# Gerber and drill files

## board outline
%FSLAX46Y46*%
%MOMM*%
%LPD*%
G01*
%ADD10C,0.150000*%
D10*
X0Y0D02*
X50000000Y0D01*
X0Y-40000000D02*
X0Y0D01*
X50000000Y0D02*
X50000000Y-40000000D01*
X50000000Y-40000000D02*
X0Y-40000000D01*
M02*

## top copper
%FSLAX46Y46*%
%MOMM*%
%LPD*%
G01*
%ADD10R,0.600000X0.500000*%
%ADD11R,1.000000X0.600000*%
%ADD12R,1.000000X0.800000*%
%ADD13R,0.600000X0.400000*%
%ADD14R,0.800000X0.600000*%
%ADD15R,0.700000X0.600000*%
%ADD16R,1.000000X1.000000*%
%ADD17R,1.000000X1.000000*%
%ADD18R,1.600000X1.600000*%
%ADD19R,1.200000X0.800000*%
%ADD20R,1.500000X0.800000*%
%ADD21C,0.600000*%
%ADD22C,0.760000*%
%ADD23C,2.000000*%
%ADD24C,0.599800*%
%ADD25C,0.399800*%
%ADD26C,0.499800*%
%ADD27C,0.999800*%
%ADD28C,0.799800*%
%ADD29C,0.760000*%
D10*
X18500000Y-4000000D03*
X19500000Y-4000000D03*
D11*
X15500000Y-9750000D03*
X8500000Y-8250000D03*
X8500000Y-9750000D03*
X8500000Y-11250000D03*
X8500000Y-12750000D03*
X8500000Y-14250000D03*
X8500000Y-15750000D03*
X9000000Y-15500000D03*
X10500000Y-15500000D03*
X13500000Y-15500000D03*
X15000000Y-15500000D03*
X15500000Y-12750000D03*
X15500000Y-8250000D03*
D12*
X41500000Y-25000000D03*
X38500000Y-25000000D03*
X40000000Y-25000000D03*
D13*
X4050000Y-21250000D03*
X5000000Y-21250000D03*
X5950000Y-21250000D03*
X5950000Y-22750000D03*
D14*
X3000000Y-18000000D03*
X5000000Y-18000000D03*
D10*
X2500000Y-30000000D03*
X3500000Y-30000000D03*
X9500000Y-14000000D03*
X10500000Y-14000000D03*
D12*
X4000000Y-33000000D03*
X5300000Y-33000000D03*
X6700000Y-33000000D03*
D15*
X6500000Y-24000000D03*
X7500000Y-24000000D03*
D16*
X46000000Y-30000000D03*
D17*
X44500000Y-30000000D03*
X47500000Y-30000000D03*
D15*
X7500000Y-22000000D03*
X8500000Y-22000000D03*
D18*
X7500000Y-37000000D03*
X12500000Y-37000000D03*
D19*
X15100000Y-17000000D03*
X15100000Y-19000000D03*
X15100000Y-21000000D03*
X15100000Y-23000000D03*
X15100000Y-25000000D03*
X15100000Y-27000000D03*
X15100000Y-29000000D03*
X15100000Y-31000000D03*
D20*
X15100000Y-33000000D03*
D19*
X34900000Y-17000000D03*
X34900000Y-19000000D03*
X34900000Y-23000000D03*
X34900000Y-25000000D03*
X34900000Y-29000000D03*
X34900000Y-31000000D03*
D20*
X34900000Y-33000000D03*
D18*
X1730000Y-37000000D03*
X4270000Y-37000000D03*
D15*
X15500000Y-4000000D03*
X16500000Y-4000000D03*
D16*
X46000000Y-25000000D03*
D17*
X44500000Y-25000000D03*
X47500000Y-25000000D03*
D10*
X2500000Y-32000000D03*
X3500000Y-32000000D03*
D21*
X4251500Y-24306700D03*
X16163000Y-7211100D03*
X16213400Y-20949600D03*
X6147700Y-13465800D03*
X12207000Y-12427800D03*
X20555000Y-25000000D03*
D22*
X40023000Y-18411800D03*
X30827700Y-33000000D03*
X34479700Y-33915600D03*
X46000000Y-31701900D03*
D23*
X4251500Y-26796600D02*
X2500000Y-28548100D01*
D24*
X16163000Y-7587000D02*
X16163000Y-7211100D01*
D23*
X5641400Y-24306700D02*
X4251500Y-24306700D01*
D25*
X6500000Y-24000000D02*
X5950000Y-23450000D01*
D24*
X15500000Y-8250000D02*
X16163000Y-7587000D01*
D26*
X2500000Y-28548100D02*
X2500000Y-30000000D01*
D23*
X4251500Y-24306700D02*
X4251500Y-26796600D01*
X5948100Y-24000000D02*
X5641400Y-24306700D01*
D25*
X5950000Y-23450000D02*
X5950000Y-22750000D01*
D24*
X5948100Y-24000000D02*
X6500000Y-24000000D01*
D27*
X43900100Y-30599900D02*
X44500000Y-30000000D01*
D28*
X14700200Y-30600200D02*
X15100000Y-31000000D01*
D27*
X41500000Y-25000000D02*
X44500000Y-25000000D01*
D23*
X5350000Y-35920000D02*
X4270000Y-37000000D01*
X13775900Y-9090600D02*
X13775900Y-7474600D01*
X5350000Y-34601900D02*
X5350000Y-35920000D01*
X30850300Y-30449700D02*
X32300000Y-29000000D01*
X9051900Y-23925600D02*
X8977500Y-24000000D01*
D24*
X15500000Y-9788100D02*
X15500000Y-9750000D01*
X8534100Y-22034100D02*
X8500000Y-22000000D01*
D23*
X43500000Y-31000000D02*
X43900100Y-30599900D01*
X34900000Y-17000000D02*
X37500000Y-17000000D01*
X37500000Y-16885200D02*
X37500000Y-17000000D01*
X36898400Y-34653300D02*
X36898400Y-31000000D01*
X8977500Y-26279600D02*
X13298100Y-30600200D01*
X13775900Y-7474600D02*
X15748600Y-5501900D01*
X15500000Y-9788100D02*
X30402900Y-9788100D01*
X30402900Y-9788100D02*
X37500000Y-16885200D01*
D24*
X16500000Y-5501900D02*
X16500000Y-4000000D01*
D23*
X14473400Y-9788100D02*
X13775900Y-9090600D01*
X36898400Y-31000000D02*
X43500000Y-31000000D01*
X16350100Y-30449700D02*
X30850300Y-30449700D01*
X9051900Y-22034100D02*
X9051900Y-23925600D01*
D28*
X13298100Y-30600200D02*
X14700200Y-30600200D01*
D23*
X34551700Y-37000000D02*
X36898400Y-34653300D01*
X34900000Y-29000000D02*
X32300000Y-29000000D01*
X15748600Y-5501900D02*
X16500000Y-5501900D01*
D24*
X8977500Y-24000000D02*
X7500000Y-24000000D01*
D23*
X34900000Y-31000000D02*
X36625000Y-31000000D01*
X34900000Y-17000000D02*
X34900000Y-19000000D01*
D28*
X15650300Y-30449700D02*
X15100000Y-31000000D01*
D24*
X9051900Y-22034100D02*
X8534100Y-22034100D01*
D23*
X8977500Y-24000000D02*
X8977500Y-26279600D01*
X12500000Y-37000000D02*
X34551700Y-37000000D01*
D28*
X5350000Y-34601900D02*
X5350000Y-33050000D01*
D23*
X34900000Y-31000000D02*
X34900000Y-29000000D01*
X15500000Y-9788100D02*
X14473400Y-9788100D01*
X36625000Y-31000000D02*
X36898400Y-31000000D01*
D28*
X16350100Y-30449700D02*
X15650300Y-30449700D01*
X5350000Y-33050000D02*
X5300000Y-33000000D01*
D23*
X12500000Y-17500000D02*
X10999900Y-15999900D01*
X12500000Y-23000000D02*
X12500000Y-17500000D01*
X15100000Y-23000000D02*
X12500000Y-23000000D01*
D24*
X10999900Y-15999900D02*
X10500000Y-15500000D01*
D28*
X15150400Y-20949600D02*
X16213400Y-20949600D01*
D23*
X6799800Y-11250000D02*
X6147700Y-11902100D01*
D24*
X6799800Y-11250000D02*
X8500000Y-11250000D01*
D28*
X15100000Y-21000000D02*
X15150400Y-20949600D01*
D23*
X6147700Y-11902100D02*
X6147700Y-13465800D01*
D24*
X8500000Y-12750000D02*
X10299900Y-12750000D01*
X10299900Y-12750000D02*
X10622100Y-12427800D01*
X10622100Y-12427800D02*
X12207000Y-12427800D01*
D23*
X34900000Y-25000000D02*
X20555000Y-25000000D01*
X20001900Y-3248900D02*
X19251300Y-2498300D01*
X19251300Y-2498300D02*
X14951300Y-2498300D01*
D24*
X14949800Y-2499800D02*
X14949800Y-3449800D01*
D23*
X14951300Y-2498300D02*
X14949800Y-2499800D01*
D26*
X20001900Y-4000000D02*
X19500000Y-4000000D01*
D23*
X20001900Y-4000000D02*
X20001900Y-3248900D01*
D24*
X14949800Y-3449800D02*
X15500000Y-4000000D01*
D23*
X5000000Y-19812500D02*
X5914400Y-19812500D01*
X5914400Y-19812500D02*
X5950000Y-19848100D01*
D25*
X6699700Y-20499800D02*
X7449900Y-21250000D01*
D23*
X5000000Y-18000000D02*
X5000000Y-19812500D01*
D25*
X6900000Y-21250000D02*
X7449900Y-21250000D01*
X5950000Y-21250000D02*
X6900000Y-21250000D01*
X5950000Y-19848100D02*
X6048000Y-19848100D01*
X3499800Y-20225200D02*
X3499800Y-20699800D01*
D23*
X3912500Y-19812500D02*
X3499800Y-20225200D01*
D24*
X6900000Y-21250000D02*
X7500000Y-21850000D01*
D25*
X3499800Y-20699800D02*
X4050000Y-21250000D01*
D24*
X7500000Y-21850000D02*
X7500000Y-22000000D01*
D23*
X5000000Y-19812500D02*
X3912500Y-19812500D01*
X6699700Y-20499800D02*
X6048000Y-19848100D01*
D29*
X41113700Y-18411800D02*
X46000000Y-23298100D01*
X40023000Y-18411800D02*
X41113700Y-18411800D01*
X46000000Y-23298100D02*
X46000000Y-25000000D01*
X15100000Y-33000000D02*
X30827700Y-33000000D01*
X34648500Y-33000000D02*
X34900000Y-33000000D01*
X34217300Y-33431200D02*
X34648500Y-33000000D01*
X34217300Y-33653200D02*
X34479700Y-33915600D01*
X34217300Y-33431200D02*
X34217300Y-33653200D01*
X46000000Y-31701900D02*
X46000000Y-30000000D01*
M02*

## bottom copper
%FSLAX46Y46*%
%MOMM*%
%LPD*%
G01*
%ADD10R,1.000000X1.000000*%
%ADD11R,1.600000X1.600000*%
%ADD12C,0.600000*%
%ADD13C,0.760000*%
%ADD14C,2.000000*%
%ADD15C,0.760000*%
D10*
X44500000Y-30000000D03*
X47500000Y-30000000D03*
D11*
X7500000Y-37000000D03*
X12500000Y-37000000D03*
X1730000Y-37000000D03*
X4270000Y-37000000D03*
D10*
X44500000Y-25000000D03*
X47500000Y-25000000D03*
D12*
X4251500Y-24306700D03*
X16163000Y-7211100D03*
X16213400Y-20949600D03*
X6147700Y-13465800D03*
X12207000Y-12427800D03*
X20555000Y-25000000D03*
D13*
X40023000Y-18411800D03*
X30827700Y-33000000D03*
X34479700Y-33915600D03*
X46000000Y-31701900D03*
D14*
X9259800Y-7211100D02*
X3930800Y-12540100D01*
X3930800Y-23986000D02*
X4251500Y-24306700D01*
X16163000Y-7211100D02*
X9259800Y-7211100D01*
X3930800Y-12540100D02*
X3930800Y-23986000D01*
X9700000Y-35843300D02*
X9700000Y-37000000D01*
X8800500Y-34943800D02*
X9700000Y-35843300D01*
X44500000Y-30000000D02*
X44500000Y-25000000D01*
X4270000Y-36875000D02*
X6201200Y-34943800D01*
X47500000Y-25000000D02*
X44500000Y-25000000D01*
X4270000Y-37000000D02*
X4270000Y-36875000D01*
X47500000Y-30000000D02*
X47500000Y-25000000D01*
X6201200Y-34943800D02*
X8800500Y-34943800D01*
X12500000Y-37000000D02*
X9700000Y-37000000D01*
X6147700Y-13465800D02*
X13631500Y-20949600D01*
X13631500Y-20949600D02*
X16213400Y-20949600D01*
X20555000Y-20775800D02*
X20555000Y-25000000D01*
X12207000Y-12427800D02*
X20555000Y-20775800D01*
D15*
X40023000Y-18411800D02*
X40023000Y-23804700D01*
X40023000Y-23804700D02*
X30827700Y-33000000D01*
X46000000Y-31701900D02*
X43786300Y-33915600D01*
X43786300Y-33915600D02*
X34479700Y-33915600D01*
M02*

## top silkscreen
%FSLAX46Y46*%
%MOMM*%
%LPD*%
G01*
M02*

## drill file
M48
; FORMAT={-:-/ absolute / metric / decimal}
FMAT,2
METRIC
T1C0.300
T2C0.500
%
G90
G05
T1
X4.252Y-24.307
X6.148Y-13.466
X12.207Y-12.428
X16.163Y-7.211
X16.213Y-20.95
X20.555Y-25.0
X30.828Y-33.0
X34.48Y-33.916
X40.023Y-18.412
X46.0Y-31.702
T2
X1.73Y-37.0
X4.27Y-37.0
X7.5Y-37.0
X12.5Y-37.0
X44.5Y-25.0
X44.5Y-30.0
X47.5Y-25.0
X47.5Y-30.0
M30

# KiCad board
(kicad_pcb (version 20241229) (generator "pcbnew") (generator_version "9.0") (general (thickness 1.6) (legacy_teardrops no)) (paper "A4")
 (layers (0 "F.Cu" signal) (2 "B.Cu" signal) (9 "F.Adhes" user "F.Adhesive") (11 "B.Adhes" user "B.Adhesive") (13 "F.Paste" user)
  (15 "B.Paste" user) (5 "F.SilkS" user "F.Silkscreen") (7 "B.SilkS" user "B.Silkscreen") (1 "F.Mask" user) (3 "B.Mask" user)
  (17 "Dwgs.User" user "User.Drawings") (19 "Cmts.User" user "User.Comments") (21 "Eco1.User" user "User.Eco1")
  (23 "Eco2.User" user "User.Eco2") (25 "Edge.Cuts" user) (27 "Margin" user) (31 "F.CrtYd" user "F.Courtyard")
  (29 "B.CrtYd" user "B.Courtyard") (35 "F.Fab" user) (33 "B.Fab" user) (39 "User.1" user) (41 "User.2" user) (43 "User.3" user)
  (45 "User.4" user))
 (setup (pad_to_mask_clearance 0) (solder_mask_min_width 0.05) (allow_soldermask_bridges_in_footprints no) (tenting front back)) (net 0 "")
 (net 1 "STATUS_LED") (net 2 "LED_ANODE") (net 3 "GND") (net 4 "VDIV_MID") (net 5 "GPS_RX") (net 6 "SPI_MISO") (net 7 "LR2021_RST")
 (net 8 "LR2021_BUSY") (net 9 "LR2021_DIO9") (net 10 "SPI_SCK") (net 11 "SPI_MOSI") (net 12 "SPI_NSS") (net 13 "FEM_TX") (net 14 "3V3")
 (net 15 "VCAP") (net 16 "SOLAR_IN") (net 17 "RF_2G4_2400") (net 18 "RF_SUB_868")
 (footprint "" (layer "F.Cu") (at 19 4)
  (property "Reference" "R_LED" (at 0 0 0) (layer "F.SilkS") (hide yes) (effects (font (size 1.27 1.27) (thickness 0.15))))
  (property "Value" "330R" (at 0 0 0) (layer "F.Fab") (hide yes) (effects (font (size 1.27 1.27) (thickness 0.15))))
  (pad "1" smd rect (at -0.5 0) (size 0.6 0.5) (layers "F.Cu" "F.Mask") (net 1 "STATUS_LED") (thermal_bridge_angle 45))
  (pad "2" smd rect (at 0.5 0) (size 0.6 0.5) (layers "F.Cu" "F.Mask") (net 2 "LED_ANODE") (thermal_bridge_angle 45)))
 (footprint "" (layer "F.Cu") (at 12 12)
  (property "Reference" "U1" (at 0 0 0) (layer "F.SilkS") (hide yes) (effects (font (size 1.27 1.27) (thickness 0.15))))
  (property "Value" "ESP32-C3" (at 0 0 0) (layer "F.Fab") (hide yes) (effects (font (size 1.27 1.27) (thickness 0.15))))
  (pad "GND" smd rect (at 3.5 -2.25) (size 1 0.6) (layers "F.Cu" "F.Mask") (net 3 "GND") (thermal_bridge_angle 45))
  (pad "GPIO0" smd rect (at -3.5 -3.75) (size 1 0.6) (layers "F.Cu" "F.Mask") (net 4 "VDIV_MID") (thermal_bridge_angle 45))
  (pad "GPIO1" smd rect (at -3.5 -2.25) (size 1 0.6) (layers "F.Cu" "F.Mask") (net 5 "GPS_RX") (thermal_bridge_angle 45))
  (pad "GPIO2" smd rect (at -3.5 -0.75) (size 1 0.6) (layers "F.Cu" "F.Mask") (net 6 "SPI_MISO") (thermal_bridge_angle 45))
  (pad "GPIO3" smd rect (at -3.5 0.75) (size 1 0.6) (layers "F.Cu" "F.Mask") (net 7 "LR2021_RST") (thermal_bridge_angle 45))
  (pad "GPIO4" smd rect (at -3.5 2.25) (size 1 0.6) (layers "F.Cu" "F.Mask") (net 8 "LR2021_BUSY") (thermal_bridge_angle 45))
  (pad "GPIO5" smd rect (at -3.5 3.75) (size 1 0.6) (layers "F.Cu" "F.Mask") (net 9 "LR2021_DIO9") (thermal_bridge_angle 45))
  (pad "GPIO6" smd rect (at -3 3.5) (size 1 0.6) (layers "F.Cu" "F.Mask") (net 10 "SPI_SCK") (thermal_bridge_angle 45))
  (pad "GPIO7" smd rect (at -1.5 3.5) (size 1 0.6) (layers "F.Cu" "F.Mask") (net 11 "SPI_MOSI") (thermal_bridge_angle 45))
  (pad "GPIO9" smd rect (at 1.5 3.5) (size 1 0.6) (layers "F.Cu" "F.Mask") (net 1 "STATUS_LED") (thermal_bridge_angle 45))
  (pad "GPIO10" smd rect (at 3 3.5) (size 1 0.6) (layers "F.Cu" "F.Mask") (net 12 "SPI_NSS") (thermal_bridge_angle 45))
  (pad "GPIO19" smd rect (at 3.5 0.75) (size 1 0.6) (layers "F.Cu" "F.Mask") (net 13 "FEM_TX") (thermal_bridge_angle 45))
  (pad "VCC" smd rect (at 3.5 -3.75) (size 1 0.6) (layers "F.Cu" "F.Mask") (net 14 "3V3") (thermal_bridge_angle 45)))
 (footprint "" (layer "F.Cu") (at 40 25)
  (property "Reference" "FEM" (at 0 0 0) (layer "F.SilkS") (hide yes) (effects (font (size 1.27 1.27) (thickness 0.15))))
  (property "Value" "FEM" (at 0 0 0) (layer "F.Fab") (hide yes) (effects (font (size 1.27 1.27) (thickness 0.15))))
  (pad "GND" smd rect (at 1.5 0) (size 1 0.8) (layers "F.Cu" "F.Mask") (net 3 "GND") (thermal_bridge_angle 45))
  (pad "TX" smd rect (at -1.5 0) (size 1 0.8) (layers "F.Cu" "F.Mask") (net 13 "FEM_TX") (thermal_bridge_angle 45))
  (pad "VCC" smd rect (at 0 0) (size 1 0.8) (layers "F.Cu" "F.Mask") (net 14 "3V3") (thermal_bridge_angle 45)))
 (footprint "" (layer "F.Cu") (at 5 22)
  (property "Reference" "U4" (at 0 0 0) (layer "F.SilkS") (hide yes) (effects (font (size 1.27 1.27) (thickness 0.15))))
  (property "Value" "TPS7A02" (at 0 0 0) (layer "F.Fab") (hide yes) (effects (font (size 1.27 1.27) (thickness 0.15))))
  (pad "1" smd rect (at -0.95 -0.75) (size 0.6 0.4) (layers "F.Cu" "F.Mask") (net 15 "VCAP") (thermal_bridge_angle 45))
  (pad "2" smd rect (at 0 -0.75) (size 0.6 0.4) (layers "F.Cu" "F.Mask") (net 3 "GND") (thermal_bridge_angle 45))
  (pad "3" smd rect (at 0.95 -0.75) (size 0.6 0.4) (layers "F.Cu" "F.Mask") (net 15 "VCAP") (thermal_bridge_angle 45))
  (pad "4" smd rect (at 0.95 0.75) (size 0.6 0.4) (layers "F.Cu" "F.Mask") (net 14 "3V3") (thermal_bridge_angle 45)))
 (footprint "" (layer "F.Cu") (at 4 18)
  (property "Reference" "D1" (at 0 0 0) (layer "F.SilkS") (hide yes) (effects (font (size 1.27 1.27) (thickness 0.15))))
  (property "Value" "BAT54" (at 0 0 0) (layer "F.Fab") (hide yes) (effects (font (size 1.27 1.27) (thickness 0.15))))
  (pad "A" smd rect (at -1 0) (size 0.8 0.6) (layers "F.Cu" "F.Mask") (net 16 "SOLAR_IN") (thermal_bridge_angle 45))
  (pad "K" smd rect (at 1 0) (size 0.8 0.6) (layers "F.Cu" "F.Mask") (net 15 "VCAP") (thermal_bridge_angle 45)))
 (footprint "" (layer "F.Cu") (at 3 30)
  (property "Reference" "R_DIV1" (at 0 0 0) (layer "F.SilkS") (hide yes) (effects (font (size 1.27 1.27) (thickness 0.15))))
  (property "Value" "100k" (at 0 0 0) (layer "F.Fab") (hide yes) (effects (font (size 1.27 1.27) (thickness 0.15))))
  (pad "1" smd rect (at -0.5 0) (size 0.6 0.5) (layers "F.Cu" "F.Mask") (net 14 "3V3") (thermal_bridge_angle 45))
  (pad "2" smd rect (at 0.5 0) (size 0.6 0.5) (layers "F.Cu" "F.Mask") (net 4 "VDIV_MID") (thermal_bridge_angle 45)))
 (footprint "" (layer "F.Cu") (at 10 14)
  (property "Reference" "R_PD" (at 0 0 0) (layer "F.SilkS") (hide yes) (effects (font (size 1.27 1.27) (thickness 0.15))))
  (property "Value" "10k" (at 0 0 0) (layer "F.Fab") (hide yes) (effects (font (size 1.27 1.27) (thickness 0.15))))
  (pad "1" smd rect (at -0.5 0) (size 0.6 0.5) (layers "F.Cu" "F.Mask") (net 3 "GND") (thermal_bridge_angle 45))
  (pad "2" smd rect (at 0.5 0) (size 0.6 0.5) (layers "F.Cu" "F.Mask") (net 6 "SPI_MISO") (thermal_bridge_angle 45)))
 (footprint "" (layer "F.Cu") (at 6 33)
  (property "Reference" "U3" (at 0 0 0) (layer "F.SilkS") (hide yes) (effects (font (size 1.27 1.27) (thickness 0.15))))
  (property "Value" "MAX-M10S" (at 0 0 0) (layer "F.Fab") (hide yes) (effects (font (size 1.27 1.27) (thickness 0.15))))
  (pad "1" smd rect (at -2 0) (size 1 0.8) (layers "F.Cu" "F.Mask") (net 14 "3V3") (thermal_bridge_angle 45))
  (pad "2" smd rect (at -0.7 0) (size 1 0.8) (layers "F.Cu" "F.Mask") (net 3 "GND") (thermal_bridge_angle 45))
  (pad "3" smd rect (at 0.7 0) (size 1 0.8) (layers "F.Cu" "F.Mask") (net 5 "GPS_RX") (thermal_bridge_angle 45)))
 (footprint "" (layer "F.Cu") (at 7 24)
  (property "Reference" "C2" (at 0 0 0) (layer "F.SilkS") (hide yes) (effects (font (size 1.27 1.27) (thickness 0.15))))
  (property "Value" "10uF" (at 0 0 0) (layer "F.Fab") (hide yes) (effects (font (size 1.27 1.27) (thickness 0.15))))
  (pad "1" smd rect (at -0.5 0) (size 0.7 0.6) (layers "F.Cu" "F.Mask") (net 14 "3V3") (thermal_bridge_angle 45))
  (pad "2" smd rect (at 0.5 0) (size 0.7 0.6) (layers "F.Cu" "F.Mask") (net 3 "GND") (thermal_bridge_angle 45)))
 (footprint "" (layer "F.Cu") (at 46 30)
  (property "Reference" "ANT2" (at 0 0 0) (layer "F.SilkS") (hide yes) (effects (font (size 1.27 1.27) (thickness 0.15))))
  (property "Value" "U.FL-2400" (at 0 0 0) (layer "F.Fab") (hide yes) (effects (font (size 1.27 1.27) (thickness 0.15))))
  (pad "1" smd rect (at 0 0) (size 1 1) (layers "F.Cu" "F.Mask") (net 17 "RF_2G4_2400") (thermal_bridge_angle 45))
  (pad "2" thru_hole rect (at -1.5 0) (size 1 1) (drill 0.5) (layers "*.Cu" "*.Mask") (remove_unused_layers no) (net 3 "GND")
   (thermal_bridge_angle 45))
  (pad "3" thru_hole rect (at 1.5 0) (size 1 1) (drill 0.5) (layers "*.Cu" "*.Mask") (remove_unused_layers no) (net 3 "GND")
   (thermal_bridge_angle 45)))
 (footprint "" (layer "F.Cu") (at 8 22)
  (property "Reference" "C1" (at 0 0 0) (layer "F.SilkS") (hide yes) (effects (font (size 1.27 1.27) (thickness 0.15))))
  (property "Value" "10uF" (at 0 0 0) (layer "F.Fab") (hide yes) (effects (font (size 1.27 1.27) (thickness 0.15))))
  (pad "1" smd rect (at -0.5 0) (size 0.7 0.6) (layers "F.Cu" "F.Mask") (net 15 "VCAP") (thermal_bridge_angle 45))
  (pad "2" smd rect (at 0.5 0) (size 0.7 0.6) (layers "F.Cu" "F.Mask") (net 3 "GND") (thermal_bridge_angle 45)))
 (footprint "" (layer "F.Cu") (at 10 37)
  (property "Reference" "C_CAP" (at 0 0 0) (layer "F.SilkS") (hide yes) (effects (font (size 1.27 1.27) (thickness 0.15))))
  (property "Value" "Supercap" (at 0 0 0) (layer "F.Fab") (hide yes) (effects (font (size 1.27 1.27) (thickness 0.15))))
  (pad "1" thru_hole rect (at -2.5 0) (size 1.6 1.6) (drill 0.5) (layers "*.Cu" "*.Mask") (remove_unused_layers no) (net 15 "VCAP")
   (thermal_bridge_angle 45))
  (pad "2" thru_hole rect (at 2.5 0) (size 1.6 1.6) (drill 0.5) (layers "*.Cu" "*.Mask") (remove_unused_layers no) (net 3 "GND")
   (thermal_bridge_angle 45)))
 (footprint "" (layer "F.Cu") (at 25 25)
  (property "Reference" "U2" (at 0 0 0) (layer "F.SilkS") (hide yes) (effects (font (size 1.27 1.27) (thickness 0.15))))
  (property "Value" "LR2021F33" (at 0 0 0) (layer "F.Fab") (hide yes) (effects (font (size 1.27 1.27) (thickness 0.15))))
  (pad "1" smd rect (at -9.9 -8) (size 1.2 0.8) (layers "F.Cu" "F.Mask") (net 14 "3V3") (thermal_bridge_angle 45))
  (pad "2" smd rect (at -9.9 -6) (size 1.2 0.8) (layers "F.Cu" "F.Mask") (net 3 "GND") (thermal_bridge_angle 45))
  (pad "3" smd rect (at -9.9 -4) (size 1.2 0.8) (layers "F.Cu" "F.Mask") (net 6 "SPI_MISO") (thermal_bridge_angle 45))
  (pad "4" smd rect (at -9.9 -2) (size 1.2 0.8) (layers "F.Cu" "F.Mask") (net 11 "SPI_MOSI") (thermal_bridge_angle 45))
  (pad "5" smd rect (at -9.9 0) (size 1.2 0.8) (layers "F.Cu" "F.Mask") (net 10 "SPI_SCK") (thermal_bridge_angle 45))
  (pad "6" smd rect (at -9.9 2) (size 1.2 0.8) (layers "F.Cu" "F.Mask") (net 12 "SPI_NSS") (thermal_bridge_angle 45))
  (pad "7" smd rect (at -9.9 4) (size 1.2 0.8) (layers "F.Cu" "F.Mask") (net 8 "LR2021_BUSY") (thermal_bridge_angle 45))
  (pad "8" smd rect (at -9.9 6) (size 1.2 0.8) (layers "F.Cu" "F.Mask") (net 3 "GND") (thermal_bridge_angle 45))
  (pad "9" smd rect (at -9.9 8) (size 1.5 0.8) (layers "F.Cu" "F.Mask") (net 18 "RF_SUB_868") (thermal_bridge_angle 45))
  (pad "10" smd rect (at 9.9 -8) (size 1.2 0.8) (layers "F.Cu" "F.Mask") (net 3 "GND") (thermal_bridge_angle 45))
  (pad "11" smd rect (at 9.9 -6) (size 1.2 0.8) (layers "F.Cu" "F.Mask") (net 3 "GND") (thermal_bridge_angle 45))
  (pad "13" smd rect (at 9.9 -2) (size 1.2 0.8) (layers "F.Cu" "F.Mask") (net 9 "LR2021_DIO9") (thermal_bridge_angle 45))
  (pad "14" smd rect (at 9.9 0) (size 1.2 0.8) (layers "F.Cu" "F.Mask") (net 7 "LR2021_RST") (thermal_bridge_angle 45))
  (pad "16" smd rect (at 9.9 4) (size 1.2 0.8) (layers "F.Cu" "F.Mask") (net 3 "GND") (thermal_bridge_angle 45))
  (pad "17" smd rect (at 9.9 6) (size 1.2 0.8) (layers "F.Cu" "F.Mask") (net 3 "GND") (thermal_bridge_angle 45))
  (pad "18" smd rect (at 9.9 8) (size 1.5 0.8) (layers "F.Cu" "F.Mask") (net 17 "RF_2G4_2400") (thermal_bridge_angle 45)))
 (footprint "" (layer "F.Cu") (at 3 37)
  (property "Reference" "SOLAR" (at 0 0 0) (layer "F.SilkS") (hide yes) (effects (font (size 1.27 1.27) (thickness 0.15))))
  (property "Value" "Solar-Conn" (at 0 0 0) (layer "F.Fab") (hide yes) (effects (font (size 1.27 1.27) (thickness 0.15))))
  (pad "1" thru_hole rect (at -1.27 0) (size 1.6 1.6) (drill 0.5) (layers "*.Cu" "*.Mask") (remove_unused_layers no) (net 16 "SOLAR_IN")
   (thermal_bridge_angle 45))
  (pad "2" thru_hole rect (at 1.27 0) (size 1.6 1.6) (drill 0.5) (layers "*.Cu" "*.Mask") (remove_unused_layers no) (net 3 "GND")
   (thermal_bridge_angle 45)))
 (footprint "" (layer "F.Cu") (at 16 4)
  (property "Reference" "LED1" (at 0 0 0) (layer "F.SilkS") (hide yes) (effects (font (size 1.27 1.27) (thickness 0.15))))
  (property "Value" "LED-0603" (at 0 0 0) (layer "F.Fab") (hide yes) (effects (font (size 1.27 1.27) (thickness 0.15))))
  (pad "A" smd rect (at -0.5 0) (size 0.7 0.6) (layers "F.Cu" "F.Mask") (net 2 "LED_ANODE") (thermal_bridge_angle 45))
  (pad "K" smd rect (at 0.5 0) (size 0.7 0.6) (layers "F.Cu" "F.Mask") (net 3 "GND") (thermal_bridge_angle 45)))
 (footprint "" (layer "F.Cu") (at 46 25)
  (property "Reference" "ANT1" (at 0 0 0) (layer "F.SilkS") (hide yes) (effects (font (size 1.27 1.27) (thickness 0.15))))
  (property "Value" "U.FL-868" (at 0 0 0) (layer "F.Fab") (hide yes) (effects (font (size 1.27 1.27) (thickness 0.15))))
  (pad "1" smd rect (at 0 0) (size 1 1) (layers "F.Cu" "F.Mask") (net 18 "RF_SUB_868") (thermal_bridge_angle 45))
  (pad "2" thru_hole rect (at -1.5 0) (size 1 1) (drill 0.5) (layers "*.Cu" "*.Mask") (remove_unused_layers no) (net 3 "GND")
   (thermal_bridge_angle 45))
  (pad "3" thru_hole rect (at 1.5 0) (size 1 1) (drill 0.5) (layers "*.Cu" "*.Mask") (remove_unused_layers no) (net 3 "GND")
   (thermal_bridge_angle 45)))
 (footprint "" (layer "F.Cu") (at 3 32)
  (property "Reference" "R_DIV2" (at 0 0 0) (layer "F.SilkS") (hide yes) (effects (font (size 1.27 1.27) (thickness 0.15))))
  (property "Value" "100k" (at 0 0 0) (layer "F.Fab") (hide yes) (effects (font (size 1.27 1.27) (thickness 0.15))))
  (pad "1" smd rect (at -0.5 0) (size 0.6 0.5) (layers "F.Cu" "F.Mask") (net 4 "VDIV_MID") (thermal_bridge_angle 45))
  (pad "2" smd rect (at 0.5 0) (size 0.6 0.5) (layers "F.Cu" "F.Mask") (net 3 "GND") (thermal_bridge_angle 45)))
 (gr_line (start 0 0) (end 50 0) (stroke (width 0.15) (type default)) (layer "Edge.Cuts"))
 (gr_line (start 0 40) (end 0 0) (stroke (width 0.15) (type default)) (layer "Edge.Cuts"))
 (gr_line (start 50 0) (end 50 40) (stroke (width 0.15) (type default)) (layer "Edge.Cuts"))
 (gr_line (start 50 40) (end 0 40) (stroke (width 0.15) (type default)) (layer "Edge.Cuts"))
 (segment (start 4.2515 26.7966) (end 2.5 28.5481) (width 2) (layer "F.Cu") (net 14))
 (segment (start 16.163 7.587) (end 16.163 7.2111) (width 0.5998) (layer "F.Cu") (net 14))
 (segment (start 5.6414 24.3067) (end 4.2515 24.3067) (width 2) (layer "F.Cu") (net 14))
 (segment (start 6.5 24) (end 5.95 23.45) (width 0.3998) (layer "F.Cu") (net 14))
 (segment (start 15.5 8.25) (end 16.163 7.587) (width 0.5998) (layer "F.Cu") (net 14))
 (segment (start 2.5 28.5481) (end 2.5 30) (width 0.4998) (layer "F.Cu") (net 14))
 (segment (start 4.2515 24.3067) (end 4.2515 26.7966) (width 2) (layer "F.Cu") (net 14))
 (segment (start 5.9481 24) (end 5.6414 24.3067) (width 2) (layer "F.Cu") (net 14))
 (segment (start 5.95 23.45) (end 5.95 22.75) (width 0.3998) (layer "F.Cu") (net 14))
 (segment (start 5.9481 24) (end 6.5 24) (width 0.5998) (layer "F.Cu") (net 14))
 (via (at 4.2515 24.3067) (size 0.6) (drill 0.3) (layers "F.Cu" "B.Cu") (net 14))
 (via (at 16.163 7.2111) (size 0.6) (drill 0.3) (layers "F.Cu" "B.Cu") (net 14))
 (segment (start 9.2598 7.2111) (end 3.9308 12.5401) (width 2) (layer "B.Cu") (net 14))
 (segment (start 3.9308 23.986) (end 4.2515 24.3067) (width 2) (layer "B.Cu") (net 14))
 (segment (start 16.163 7.2111) (end 9.2598 7.2111) (width 2) (layer "B.Cu") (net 14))
 (segment (start 3.9308 12.5401) (end 3.9308 23.986) (width 2) (layer "B.Cu") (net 14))
 (segment (start 43.9001 30.5999) (end 44.5 30) (width 0.9998) (layer "F.Cu") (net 3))
 (segment (start 14.7002 30.6002) (end 15.1 31) (width 0.7998) (layer "F.Cu") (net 3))
 (segment (start 41.5 25) (end 44.5 25) (width 0.9998) (layer "F.Cu") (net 3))
 (segment (start 5.35 35.92) (end 4.27 37) (width 2) (layer "F.Cu") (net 3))
 (segment (start 13.7759 9.0906) (end 13.7759 7.4746) (width 2) (layer "F.Cu") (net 3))
 (segment (start 5.35 34.6019) (end 5.35 35.92) (width 2) (layer "F.Cu") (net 3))
 (segment (start 30.8503 30.4497) (end 32.3 29) (width 2) (layer "F.Cu") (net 3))
 (segment (start 9.0519 23.9256) (end 8.9775 24) (width 2) (layer "F.Cu") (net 3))
 (segment (start 15.5 9.7881) (end 15.5 9.75) (width 0.5998) (layer "F.Cu") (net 3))
 (segment (start 8.5341 22.0341) (end 8.5 22) (width 0.5998) (layer "F.Cu") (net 3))
 (segment (start 43.5 31) (end 43.9001 30.5999) (width 2) (layer "F.Cu") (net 3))
 (segment (start 34.9 17) (end 37.5 17) (width 2) (layer "F.Cu") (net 3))
 (segment (start 37.5 16.8852) (end 37.5 17) (width 2) (layer "F.Cu") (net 3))
 (segment (start 36.8984 34.6533) (end 36.8984 31) (width 2) (layer "F.Cu") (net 3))
 (segment (start 8.9775 26.2796) (end 13.2981 30.6002) (width 2) (layer "F.Cu") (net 3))
 (segment (start 13.7759 7.4746) (end 15.7486 5.5019) (width 2) (layer "F.Cu") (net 3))
 (segment (start 15.5 9.7881) (end 30.4029 9.7881) (width 2) (layer "F.Cu") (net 3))
 (segment (start 30.4029 9.7881) (end 37.5 16.8852) (width 2) (layer "F.Cu") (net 3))
 (segment (start 16.5 5.5019) (end 16.5 4) (width 0.5998) (layer "F.Cu") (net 3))
 (segment (start 14.4734 9.7881) (end 13.7759 9.0906) (width 2) (layer "F.Cu") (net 3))
 (segment (start 36.8984 31) (end 43.5 31) (width 2) (layer "F.Cu") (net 3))
 (segment (start 16.3501 30.4497) (end 30.8503 30.4497) (width 2) (layer "F.Cu") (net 3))
 (segment (start 9.0519 22.0341) (end 9.0519 23.9256) (width 2) (layer "F.Cu") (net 3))
 (segment (start 13.2981 30.6002) (end 14.7002 30.6002) (width 0.7998) (layer "F.Cu") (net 3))
 (segment (start 34.5517 37) (end 36.8984 34.6533) (width 2) (layer "F.Cu") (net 3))
 (segment (start 34.9 29) (end 32.3 29) (width 2) (layer "F.Cu") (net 3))
 (segment (start 15.7486 5.5019) (end 16.5 5.5019) (width 2) (layer "F.Cu") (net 3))
 (segment (start 8.9775 24) (end 7.5 24) (width 0.5998) (layer "F.Cu") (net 3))
 (segment (start 34.9 31) (end 36.625 31) (width 2) (layer "F.Cu") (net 3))
 (segment (start 34.9 17) (end 34.9 19) (width 2) (layer "F.Cu") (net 3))
 (segment (start 15.6503 30.4497) (end 15.1 31) (width 0.7998) (layer "F.Cu") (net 3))
 (segment (start 9.0519 22.0341) (end 8.5341 22.0341) (width 0.5998) (layer "F.Cu") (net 3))
 (segment (start 8.9775 24) (end 8.9775 26.2796) (width 2) (layer "F.Cu") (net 3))
 (segment (start 12.5 37) (end 34.5517 37) (width 2) (layer "F.Cu") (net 3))
 (segment (start 5.35 34.6019) (end 5.35 33.05) (width 0.7998) (layer "F.Cu") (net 3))
 (segment (start 34.9 31) (end 34.9 29) (width 2) (layer "F.Cu") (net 3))
 (segment (start 15.5 9.7881) (end 14.4734 9.7881) (width 2) (layer "F.Cu") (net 3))
 (segment (start 36.625 31) (end 36.8984 31) (width 2) (layer "F.Cu") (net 3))
 (segment (start 16.3501 30.4497) (end 15.6503 30.4497) (width 0.7998) (layer "F.Cu") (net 3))
 (segment (start 5.35 33.05) (end 5.3 33) (width 0.7998) (layer "F.Cu") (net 3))
 (segment (start 9.7 35.8433) (end 9.7 37) (width 2) (layer "B.Cu") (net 3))
 (segment (start 8.8005 34.9438) (end 9.7 35.8433) (width 2) (layer "B.Cu") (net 3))
 (segment (start 44.5 30) (end 44.5 25) (width 2) (layer "B.Cu") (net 3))
 (segment (start 4.27 36.875) (end 6.2012 34.9438) (width 2) (layer "B.Cu") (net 3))
 (segment (start 47.5 25) (end 44.5 25) (width 2) (layer "B.Cu") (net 3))
 (segment (start 4.27 37) (end 4.27 36.875) (width 2) (layer "B.Cu") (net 3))
 (segment (start 47.5 30) (end 47.5 25) (width 2) (layer "B.Cu") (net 3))
 (segment (start 6.2012 34.9438) (end 8.8005 34.9438) (width 2) (layer "B.Cu") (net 3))
 (segment (start 12.5 37) (end 9.7 37) (width 2) (layer "B.Cu") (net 3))
 (segment (start 12.5 17.5) (end 10.9999 15.9999) (width 2) (layer "F.Cu") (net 11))
 (segment (start 12.5 23) (end 12.5 17.5) (width 2) (layer "F.Cu") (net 11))
 (segment (start 15.1 23) (end 12.5 23) (width 2) (layer "F.Cu") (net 11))
 (segment (start 10.9999 15.9999) (end 10.5 15.5) (width 0.5998) (layer "F.Cu") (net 11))
 (segment (start 15.1504 20.9496) (end 16.2134 20.9496) (width 0.7998) (layer "F.Cu") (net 6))
 (segment (start 6.7998 11.25) (end 6.1477 11.9021) (width 2) (layer "F.Cu") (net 6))
 (segment (start 6.7998 11.25) (end 8.5 11.25) (width 0.5998) (layer "F.Cu") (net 6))
 (segment (start 15.1 21) (end 15.1504 20.9496) (width 0.7998) (layer "F.Cu") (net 6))
 (segment (start 6.1477 11.9021) (end 6.1477 13.4658) (width 2) (layer "F.Cu") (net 6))
 (via (at 16.2134 20.9496) (size 0.6) (drill 0.3) (layers "F.Cu" "B.Cu") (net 6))
 (via (at 6.1477 13.4658) (size 0.6) (drill 0.3) (layers "F.Cu" "B.Cu") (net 6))
 (segment (start 6.1477 13.4658) (end 13.6315 20.9496) (width 2) (layer "B.Cu") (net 6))
 (segment (start 13.6315 20.9496) (end 16.2134 20.9496) (width 2) (layer "B.Cu") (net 6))
 (segment (start 8.5 12.75) (end 10.2999 12.75) (width 0.5998) (layer "F.Cu") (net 7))
 (segment (start 10.2999 12.75) (end 10.6221 12.4278) (width 0.5998) (layer "F.Cu") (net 7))
 (segment (start 10.6221 12.4278) (end 12.207 12.4278) (width 0.5998) (layer "F.Cu") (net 7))
 (segment (start 34.9 25) (end 20.555 25) (width 2) (layer "F.Cu") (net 7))
 (via (at 12.207 12.4278) (size 0.6) (drill 0.3) (layers "F.Cu" "B.Cu") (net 7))
 (via (at 20.555 25) (size 0.6) (drill 0.3) (layers "F.Cu" "B.Cu") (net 7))
 (segment (start 20.555 20.7758) (end 20.555 25) (width 2) (layer "B.Cu") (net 7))
 (segment (start 12.207 12.4278) (end 20.555 20.7758) (width 2) (layer "B.Cu") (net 7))
 (segment (start 20.0019 3.2489) (end 19.2513 2.4983) (width 2) (layer "F.Cu") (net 2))
 (segment (start 19.2513 2.4983) (end 14.9513 2.4983) (width 2) (layer "F.Cu") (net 2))
 (segment (start 14.9498 2.4998) (end 14.9498 3.4498) (width 0.5998) (layer "F.Cu") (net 2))
 (segment (start 14.9513 2.4983) (end 14.9498 2.4998) (width 2) (layer "F.Cu") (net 2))
 (segment (start 20.0019 4) (end 19.5 4) (width 0.4998) (layer "F.Cu") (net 2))
 (segment (start 20.0019 4) (end 20.0019 3.2489) (width 2) (layer "F.Cu") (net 2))
 (segment (start 14.9498 3.4498) (end 15.5 4) (width 0.5998) (layer "F.Cu") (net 2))
 (segment (start 5 19.8125) (end 5.9144 19.8125) (width 2) (layer "F.Cu") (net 15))
 (segment (start 5.9144 19.8125) (end 5.95 19.8481) (width 2) (layer "F.Cu") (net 15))
 (segment (start 6.6997 20.4998) (end 7.4499 21.25) (width 0.3998) (layer "F.Cu") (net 15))
 (segment (start 5 18) (end 5 19.8125) (width 2) (layer "F.Cu") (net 15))
 (segment (start 6.9 21.25) (end 7.4499 21.25) (width 0.3998) (layer "F.Cu") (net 15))
 (segment (start 5.95 21.25) (end 6.9 21.25) (width 0.3998) (layer "F.Cu") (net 15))
 (segment (start 5.95 19.8481) (end 6.048 19.8481) (width 0.3998) (layer "F.Cu") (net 15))
 (segment (start 3.4998 20.2252) (end 3.4998 20.6998) (width 0.3998) (layer "F.Cu") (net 15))
 (segment (start 3.9125 19.8125) (end 3.4998 20.2252) (width 2) (layer "F.Cu") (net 15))
 (segment (start 6.9 21.25) (end 7.5 21.85) (width 0.5998) (layer "F.Cu") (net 15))
 (segment (start 3.4998 20.6998) (end 4.05 21.25) (width 0.3998) (layer "F.Cu") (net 15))
 (segment (start 7.5 21.85) (end 7.5 22) (width 0.5998) (layer "F.Cu") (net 15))
 (segment (start 5 19.8125) (end 3.9125 19.8125) (width 2) (layer "F.Cu") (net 15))
 (segment (start 6.6997 20.4998) (end 6.048 19.8481) (width 2) (layer "F.Cu") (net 15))
 (segment (start 41.1137 18.4118) (end 46 23.2981) (width 0.76) (layer "F.Cu") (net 18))
 (segment (start 40.023 18.4118) (end 41.1137 18.4118) (width 0.76) (layer "F.Cu") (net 18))
 (segment (start 46 23.2981) (end 46 25) (width 0.76) (layer "F.Cu") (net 18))
 (segment (start 15.1 33) (end 30.8277 33) (width 0.76) (layer "F.Cu") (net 18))
 (via (at 40.023 18.4118) (size 0.76) (drill 0.3) (layers "F.Cu" "B.Cu") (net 18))
 (via (at 30.8277 33) (size 0.76) (drill 0.3) (layers "F.Cu" "B.Cu") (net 18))
 (segment (start 40.023 18.4118) (end 40.023 23.8047) (width 0.76) (layer "B.Cu") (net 18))
 (segment (start 40.023 23.8047) (end 30.8277 33) (width 0.76) (layer "B.Cu") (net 18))
 (segment (start 34.6485 33) (end 34.9 33) (width 0.76) (layer "F.Cu") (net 17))
 (segment (start 34.2173 33.4312) (end 34.6485 33) (width 0.76) (layer "F.Cu") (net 17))
 (segment (start 34.2173 33.6532) (end 34.4797 33.9156) (width 0.76) (layer "F.Cu") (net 17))
 (segment (start 34.2173 33.4312) (end 34.2173 33.6532) (width 0.76) (layer "F.Cu") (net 17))
 (segment (start 46 31.7019) (end 46 30) (width 0.76) (layer "F.Cu") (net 17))
 (via (at 34.4797 33.9156) (size 0.76) (drill 0.3) (layers "F.Cu" "B.Cu") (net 17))
 (via (at 46 31.7019) (size 0.76) (drill 0.3) (layers "F.Cu" "B.Cu") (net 17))
 (segment (start 46 31.7019) (end 43.7863 33.9156) (width 0.76) (layer "B.Cu") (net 17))
 (segment (start 43.7863 33.9156) (end 34.4797 33.9156) (width 0.76) (layer "B.Cu") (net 17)))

